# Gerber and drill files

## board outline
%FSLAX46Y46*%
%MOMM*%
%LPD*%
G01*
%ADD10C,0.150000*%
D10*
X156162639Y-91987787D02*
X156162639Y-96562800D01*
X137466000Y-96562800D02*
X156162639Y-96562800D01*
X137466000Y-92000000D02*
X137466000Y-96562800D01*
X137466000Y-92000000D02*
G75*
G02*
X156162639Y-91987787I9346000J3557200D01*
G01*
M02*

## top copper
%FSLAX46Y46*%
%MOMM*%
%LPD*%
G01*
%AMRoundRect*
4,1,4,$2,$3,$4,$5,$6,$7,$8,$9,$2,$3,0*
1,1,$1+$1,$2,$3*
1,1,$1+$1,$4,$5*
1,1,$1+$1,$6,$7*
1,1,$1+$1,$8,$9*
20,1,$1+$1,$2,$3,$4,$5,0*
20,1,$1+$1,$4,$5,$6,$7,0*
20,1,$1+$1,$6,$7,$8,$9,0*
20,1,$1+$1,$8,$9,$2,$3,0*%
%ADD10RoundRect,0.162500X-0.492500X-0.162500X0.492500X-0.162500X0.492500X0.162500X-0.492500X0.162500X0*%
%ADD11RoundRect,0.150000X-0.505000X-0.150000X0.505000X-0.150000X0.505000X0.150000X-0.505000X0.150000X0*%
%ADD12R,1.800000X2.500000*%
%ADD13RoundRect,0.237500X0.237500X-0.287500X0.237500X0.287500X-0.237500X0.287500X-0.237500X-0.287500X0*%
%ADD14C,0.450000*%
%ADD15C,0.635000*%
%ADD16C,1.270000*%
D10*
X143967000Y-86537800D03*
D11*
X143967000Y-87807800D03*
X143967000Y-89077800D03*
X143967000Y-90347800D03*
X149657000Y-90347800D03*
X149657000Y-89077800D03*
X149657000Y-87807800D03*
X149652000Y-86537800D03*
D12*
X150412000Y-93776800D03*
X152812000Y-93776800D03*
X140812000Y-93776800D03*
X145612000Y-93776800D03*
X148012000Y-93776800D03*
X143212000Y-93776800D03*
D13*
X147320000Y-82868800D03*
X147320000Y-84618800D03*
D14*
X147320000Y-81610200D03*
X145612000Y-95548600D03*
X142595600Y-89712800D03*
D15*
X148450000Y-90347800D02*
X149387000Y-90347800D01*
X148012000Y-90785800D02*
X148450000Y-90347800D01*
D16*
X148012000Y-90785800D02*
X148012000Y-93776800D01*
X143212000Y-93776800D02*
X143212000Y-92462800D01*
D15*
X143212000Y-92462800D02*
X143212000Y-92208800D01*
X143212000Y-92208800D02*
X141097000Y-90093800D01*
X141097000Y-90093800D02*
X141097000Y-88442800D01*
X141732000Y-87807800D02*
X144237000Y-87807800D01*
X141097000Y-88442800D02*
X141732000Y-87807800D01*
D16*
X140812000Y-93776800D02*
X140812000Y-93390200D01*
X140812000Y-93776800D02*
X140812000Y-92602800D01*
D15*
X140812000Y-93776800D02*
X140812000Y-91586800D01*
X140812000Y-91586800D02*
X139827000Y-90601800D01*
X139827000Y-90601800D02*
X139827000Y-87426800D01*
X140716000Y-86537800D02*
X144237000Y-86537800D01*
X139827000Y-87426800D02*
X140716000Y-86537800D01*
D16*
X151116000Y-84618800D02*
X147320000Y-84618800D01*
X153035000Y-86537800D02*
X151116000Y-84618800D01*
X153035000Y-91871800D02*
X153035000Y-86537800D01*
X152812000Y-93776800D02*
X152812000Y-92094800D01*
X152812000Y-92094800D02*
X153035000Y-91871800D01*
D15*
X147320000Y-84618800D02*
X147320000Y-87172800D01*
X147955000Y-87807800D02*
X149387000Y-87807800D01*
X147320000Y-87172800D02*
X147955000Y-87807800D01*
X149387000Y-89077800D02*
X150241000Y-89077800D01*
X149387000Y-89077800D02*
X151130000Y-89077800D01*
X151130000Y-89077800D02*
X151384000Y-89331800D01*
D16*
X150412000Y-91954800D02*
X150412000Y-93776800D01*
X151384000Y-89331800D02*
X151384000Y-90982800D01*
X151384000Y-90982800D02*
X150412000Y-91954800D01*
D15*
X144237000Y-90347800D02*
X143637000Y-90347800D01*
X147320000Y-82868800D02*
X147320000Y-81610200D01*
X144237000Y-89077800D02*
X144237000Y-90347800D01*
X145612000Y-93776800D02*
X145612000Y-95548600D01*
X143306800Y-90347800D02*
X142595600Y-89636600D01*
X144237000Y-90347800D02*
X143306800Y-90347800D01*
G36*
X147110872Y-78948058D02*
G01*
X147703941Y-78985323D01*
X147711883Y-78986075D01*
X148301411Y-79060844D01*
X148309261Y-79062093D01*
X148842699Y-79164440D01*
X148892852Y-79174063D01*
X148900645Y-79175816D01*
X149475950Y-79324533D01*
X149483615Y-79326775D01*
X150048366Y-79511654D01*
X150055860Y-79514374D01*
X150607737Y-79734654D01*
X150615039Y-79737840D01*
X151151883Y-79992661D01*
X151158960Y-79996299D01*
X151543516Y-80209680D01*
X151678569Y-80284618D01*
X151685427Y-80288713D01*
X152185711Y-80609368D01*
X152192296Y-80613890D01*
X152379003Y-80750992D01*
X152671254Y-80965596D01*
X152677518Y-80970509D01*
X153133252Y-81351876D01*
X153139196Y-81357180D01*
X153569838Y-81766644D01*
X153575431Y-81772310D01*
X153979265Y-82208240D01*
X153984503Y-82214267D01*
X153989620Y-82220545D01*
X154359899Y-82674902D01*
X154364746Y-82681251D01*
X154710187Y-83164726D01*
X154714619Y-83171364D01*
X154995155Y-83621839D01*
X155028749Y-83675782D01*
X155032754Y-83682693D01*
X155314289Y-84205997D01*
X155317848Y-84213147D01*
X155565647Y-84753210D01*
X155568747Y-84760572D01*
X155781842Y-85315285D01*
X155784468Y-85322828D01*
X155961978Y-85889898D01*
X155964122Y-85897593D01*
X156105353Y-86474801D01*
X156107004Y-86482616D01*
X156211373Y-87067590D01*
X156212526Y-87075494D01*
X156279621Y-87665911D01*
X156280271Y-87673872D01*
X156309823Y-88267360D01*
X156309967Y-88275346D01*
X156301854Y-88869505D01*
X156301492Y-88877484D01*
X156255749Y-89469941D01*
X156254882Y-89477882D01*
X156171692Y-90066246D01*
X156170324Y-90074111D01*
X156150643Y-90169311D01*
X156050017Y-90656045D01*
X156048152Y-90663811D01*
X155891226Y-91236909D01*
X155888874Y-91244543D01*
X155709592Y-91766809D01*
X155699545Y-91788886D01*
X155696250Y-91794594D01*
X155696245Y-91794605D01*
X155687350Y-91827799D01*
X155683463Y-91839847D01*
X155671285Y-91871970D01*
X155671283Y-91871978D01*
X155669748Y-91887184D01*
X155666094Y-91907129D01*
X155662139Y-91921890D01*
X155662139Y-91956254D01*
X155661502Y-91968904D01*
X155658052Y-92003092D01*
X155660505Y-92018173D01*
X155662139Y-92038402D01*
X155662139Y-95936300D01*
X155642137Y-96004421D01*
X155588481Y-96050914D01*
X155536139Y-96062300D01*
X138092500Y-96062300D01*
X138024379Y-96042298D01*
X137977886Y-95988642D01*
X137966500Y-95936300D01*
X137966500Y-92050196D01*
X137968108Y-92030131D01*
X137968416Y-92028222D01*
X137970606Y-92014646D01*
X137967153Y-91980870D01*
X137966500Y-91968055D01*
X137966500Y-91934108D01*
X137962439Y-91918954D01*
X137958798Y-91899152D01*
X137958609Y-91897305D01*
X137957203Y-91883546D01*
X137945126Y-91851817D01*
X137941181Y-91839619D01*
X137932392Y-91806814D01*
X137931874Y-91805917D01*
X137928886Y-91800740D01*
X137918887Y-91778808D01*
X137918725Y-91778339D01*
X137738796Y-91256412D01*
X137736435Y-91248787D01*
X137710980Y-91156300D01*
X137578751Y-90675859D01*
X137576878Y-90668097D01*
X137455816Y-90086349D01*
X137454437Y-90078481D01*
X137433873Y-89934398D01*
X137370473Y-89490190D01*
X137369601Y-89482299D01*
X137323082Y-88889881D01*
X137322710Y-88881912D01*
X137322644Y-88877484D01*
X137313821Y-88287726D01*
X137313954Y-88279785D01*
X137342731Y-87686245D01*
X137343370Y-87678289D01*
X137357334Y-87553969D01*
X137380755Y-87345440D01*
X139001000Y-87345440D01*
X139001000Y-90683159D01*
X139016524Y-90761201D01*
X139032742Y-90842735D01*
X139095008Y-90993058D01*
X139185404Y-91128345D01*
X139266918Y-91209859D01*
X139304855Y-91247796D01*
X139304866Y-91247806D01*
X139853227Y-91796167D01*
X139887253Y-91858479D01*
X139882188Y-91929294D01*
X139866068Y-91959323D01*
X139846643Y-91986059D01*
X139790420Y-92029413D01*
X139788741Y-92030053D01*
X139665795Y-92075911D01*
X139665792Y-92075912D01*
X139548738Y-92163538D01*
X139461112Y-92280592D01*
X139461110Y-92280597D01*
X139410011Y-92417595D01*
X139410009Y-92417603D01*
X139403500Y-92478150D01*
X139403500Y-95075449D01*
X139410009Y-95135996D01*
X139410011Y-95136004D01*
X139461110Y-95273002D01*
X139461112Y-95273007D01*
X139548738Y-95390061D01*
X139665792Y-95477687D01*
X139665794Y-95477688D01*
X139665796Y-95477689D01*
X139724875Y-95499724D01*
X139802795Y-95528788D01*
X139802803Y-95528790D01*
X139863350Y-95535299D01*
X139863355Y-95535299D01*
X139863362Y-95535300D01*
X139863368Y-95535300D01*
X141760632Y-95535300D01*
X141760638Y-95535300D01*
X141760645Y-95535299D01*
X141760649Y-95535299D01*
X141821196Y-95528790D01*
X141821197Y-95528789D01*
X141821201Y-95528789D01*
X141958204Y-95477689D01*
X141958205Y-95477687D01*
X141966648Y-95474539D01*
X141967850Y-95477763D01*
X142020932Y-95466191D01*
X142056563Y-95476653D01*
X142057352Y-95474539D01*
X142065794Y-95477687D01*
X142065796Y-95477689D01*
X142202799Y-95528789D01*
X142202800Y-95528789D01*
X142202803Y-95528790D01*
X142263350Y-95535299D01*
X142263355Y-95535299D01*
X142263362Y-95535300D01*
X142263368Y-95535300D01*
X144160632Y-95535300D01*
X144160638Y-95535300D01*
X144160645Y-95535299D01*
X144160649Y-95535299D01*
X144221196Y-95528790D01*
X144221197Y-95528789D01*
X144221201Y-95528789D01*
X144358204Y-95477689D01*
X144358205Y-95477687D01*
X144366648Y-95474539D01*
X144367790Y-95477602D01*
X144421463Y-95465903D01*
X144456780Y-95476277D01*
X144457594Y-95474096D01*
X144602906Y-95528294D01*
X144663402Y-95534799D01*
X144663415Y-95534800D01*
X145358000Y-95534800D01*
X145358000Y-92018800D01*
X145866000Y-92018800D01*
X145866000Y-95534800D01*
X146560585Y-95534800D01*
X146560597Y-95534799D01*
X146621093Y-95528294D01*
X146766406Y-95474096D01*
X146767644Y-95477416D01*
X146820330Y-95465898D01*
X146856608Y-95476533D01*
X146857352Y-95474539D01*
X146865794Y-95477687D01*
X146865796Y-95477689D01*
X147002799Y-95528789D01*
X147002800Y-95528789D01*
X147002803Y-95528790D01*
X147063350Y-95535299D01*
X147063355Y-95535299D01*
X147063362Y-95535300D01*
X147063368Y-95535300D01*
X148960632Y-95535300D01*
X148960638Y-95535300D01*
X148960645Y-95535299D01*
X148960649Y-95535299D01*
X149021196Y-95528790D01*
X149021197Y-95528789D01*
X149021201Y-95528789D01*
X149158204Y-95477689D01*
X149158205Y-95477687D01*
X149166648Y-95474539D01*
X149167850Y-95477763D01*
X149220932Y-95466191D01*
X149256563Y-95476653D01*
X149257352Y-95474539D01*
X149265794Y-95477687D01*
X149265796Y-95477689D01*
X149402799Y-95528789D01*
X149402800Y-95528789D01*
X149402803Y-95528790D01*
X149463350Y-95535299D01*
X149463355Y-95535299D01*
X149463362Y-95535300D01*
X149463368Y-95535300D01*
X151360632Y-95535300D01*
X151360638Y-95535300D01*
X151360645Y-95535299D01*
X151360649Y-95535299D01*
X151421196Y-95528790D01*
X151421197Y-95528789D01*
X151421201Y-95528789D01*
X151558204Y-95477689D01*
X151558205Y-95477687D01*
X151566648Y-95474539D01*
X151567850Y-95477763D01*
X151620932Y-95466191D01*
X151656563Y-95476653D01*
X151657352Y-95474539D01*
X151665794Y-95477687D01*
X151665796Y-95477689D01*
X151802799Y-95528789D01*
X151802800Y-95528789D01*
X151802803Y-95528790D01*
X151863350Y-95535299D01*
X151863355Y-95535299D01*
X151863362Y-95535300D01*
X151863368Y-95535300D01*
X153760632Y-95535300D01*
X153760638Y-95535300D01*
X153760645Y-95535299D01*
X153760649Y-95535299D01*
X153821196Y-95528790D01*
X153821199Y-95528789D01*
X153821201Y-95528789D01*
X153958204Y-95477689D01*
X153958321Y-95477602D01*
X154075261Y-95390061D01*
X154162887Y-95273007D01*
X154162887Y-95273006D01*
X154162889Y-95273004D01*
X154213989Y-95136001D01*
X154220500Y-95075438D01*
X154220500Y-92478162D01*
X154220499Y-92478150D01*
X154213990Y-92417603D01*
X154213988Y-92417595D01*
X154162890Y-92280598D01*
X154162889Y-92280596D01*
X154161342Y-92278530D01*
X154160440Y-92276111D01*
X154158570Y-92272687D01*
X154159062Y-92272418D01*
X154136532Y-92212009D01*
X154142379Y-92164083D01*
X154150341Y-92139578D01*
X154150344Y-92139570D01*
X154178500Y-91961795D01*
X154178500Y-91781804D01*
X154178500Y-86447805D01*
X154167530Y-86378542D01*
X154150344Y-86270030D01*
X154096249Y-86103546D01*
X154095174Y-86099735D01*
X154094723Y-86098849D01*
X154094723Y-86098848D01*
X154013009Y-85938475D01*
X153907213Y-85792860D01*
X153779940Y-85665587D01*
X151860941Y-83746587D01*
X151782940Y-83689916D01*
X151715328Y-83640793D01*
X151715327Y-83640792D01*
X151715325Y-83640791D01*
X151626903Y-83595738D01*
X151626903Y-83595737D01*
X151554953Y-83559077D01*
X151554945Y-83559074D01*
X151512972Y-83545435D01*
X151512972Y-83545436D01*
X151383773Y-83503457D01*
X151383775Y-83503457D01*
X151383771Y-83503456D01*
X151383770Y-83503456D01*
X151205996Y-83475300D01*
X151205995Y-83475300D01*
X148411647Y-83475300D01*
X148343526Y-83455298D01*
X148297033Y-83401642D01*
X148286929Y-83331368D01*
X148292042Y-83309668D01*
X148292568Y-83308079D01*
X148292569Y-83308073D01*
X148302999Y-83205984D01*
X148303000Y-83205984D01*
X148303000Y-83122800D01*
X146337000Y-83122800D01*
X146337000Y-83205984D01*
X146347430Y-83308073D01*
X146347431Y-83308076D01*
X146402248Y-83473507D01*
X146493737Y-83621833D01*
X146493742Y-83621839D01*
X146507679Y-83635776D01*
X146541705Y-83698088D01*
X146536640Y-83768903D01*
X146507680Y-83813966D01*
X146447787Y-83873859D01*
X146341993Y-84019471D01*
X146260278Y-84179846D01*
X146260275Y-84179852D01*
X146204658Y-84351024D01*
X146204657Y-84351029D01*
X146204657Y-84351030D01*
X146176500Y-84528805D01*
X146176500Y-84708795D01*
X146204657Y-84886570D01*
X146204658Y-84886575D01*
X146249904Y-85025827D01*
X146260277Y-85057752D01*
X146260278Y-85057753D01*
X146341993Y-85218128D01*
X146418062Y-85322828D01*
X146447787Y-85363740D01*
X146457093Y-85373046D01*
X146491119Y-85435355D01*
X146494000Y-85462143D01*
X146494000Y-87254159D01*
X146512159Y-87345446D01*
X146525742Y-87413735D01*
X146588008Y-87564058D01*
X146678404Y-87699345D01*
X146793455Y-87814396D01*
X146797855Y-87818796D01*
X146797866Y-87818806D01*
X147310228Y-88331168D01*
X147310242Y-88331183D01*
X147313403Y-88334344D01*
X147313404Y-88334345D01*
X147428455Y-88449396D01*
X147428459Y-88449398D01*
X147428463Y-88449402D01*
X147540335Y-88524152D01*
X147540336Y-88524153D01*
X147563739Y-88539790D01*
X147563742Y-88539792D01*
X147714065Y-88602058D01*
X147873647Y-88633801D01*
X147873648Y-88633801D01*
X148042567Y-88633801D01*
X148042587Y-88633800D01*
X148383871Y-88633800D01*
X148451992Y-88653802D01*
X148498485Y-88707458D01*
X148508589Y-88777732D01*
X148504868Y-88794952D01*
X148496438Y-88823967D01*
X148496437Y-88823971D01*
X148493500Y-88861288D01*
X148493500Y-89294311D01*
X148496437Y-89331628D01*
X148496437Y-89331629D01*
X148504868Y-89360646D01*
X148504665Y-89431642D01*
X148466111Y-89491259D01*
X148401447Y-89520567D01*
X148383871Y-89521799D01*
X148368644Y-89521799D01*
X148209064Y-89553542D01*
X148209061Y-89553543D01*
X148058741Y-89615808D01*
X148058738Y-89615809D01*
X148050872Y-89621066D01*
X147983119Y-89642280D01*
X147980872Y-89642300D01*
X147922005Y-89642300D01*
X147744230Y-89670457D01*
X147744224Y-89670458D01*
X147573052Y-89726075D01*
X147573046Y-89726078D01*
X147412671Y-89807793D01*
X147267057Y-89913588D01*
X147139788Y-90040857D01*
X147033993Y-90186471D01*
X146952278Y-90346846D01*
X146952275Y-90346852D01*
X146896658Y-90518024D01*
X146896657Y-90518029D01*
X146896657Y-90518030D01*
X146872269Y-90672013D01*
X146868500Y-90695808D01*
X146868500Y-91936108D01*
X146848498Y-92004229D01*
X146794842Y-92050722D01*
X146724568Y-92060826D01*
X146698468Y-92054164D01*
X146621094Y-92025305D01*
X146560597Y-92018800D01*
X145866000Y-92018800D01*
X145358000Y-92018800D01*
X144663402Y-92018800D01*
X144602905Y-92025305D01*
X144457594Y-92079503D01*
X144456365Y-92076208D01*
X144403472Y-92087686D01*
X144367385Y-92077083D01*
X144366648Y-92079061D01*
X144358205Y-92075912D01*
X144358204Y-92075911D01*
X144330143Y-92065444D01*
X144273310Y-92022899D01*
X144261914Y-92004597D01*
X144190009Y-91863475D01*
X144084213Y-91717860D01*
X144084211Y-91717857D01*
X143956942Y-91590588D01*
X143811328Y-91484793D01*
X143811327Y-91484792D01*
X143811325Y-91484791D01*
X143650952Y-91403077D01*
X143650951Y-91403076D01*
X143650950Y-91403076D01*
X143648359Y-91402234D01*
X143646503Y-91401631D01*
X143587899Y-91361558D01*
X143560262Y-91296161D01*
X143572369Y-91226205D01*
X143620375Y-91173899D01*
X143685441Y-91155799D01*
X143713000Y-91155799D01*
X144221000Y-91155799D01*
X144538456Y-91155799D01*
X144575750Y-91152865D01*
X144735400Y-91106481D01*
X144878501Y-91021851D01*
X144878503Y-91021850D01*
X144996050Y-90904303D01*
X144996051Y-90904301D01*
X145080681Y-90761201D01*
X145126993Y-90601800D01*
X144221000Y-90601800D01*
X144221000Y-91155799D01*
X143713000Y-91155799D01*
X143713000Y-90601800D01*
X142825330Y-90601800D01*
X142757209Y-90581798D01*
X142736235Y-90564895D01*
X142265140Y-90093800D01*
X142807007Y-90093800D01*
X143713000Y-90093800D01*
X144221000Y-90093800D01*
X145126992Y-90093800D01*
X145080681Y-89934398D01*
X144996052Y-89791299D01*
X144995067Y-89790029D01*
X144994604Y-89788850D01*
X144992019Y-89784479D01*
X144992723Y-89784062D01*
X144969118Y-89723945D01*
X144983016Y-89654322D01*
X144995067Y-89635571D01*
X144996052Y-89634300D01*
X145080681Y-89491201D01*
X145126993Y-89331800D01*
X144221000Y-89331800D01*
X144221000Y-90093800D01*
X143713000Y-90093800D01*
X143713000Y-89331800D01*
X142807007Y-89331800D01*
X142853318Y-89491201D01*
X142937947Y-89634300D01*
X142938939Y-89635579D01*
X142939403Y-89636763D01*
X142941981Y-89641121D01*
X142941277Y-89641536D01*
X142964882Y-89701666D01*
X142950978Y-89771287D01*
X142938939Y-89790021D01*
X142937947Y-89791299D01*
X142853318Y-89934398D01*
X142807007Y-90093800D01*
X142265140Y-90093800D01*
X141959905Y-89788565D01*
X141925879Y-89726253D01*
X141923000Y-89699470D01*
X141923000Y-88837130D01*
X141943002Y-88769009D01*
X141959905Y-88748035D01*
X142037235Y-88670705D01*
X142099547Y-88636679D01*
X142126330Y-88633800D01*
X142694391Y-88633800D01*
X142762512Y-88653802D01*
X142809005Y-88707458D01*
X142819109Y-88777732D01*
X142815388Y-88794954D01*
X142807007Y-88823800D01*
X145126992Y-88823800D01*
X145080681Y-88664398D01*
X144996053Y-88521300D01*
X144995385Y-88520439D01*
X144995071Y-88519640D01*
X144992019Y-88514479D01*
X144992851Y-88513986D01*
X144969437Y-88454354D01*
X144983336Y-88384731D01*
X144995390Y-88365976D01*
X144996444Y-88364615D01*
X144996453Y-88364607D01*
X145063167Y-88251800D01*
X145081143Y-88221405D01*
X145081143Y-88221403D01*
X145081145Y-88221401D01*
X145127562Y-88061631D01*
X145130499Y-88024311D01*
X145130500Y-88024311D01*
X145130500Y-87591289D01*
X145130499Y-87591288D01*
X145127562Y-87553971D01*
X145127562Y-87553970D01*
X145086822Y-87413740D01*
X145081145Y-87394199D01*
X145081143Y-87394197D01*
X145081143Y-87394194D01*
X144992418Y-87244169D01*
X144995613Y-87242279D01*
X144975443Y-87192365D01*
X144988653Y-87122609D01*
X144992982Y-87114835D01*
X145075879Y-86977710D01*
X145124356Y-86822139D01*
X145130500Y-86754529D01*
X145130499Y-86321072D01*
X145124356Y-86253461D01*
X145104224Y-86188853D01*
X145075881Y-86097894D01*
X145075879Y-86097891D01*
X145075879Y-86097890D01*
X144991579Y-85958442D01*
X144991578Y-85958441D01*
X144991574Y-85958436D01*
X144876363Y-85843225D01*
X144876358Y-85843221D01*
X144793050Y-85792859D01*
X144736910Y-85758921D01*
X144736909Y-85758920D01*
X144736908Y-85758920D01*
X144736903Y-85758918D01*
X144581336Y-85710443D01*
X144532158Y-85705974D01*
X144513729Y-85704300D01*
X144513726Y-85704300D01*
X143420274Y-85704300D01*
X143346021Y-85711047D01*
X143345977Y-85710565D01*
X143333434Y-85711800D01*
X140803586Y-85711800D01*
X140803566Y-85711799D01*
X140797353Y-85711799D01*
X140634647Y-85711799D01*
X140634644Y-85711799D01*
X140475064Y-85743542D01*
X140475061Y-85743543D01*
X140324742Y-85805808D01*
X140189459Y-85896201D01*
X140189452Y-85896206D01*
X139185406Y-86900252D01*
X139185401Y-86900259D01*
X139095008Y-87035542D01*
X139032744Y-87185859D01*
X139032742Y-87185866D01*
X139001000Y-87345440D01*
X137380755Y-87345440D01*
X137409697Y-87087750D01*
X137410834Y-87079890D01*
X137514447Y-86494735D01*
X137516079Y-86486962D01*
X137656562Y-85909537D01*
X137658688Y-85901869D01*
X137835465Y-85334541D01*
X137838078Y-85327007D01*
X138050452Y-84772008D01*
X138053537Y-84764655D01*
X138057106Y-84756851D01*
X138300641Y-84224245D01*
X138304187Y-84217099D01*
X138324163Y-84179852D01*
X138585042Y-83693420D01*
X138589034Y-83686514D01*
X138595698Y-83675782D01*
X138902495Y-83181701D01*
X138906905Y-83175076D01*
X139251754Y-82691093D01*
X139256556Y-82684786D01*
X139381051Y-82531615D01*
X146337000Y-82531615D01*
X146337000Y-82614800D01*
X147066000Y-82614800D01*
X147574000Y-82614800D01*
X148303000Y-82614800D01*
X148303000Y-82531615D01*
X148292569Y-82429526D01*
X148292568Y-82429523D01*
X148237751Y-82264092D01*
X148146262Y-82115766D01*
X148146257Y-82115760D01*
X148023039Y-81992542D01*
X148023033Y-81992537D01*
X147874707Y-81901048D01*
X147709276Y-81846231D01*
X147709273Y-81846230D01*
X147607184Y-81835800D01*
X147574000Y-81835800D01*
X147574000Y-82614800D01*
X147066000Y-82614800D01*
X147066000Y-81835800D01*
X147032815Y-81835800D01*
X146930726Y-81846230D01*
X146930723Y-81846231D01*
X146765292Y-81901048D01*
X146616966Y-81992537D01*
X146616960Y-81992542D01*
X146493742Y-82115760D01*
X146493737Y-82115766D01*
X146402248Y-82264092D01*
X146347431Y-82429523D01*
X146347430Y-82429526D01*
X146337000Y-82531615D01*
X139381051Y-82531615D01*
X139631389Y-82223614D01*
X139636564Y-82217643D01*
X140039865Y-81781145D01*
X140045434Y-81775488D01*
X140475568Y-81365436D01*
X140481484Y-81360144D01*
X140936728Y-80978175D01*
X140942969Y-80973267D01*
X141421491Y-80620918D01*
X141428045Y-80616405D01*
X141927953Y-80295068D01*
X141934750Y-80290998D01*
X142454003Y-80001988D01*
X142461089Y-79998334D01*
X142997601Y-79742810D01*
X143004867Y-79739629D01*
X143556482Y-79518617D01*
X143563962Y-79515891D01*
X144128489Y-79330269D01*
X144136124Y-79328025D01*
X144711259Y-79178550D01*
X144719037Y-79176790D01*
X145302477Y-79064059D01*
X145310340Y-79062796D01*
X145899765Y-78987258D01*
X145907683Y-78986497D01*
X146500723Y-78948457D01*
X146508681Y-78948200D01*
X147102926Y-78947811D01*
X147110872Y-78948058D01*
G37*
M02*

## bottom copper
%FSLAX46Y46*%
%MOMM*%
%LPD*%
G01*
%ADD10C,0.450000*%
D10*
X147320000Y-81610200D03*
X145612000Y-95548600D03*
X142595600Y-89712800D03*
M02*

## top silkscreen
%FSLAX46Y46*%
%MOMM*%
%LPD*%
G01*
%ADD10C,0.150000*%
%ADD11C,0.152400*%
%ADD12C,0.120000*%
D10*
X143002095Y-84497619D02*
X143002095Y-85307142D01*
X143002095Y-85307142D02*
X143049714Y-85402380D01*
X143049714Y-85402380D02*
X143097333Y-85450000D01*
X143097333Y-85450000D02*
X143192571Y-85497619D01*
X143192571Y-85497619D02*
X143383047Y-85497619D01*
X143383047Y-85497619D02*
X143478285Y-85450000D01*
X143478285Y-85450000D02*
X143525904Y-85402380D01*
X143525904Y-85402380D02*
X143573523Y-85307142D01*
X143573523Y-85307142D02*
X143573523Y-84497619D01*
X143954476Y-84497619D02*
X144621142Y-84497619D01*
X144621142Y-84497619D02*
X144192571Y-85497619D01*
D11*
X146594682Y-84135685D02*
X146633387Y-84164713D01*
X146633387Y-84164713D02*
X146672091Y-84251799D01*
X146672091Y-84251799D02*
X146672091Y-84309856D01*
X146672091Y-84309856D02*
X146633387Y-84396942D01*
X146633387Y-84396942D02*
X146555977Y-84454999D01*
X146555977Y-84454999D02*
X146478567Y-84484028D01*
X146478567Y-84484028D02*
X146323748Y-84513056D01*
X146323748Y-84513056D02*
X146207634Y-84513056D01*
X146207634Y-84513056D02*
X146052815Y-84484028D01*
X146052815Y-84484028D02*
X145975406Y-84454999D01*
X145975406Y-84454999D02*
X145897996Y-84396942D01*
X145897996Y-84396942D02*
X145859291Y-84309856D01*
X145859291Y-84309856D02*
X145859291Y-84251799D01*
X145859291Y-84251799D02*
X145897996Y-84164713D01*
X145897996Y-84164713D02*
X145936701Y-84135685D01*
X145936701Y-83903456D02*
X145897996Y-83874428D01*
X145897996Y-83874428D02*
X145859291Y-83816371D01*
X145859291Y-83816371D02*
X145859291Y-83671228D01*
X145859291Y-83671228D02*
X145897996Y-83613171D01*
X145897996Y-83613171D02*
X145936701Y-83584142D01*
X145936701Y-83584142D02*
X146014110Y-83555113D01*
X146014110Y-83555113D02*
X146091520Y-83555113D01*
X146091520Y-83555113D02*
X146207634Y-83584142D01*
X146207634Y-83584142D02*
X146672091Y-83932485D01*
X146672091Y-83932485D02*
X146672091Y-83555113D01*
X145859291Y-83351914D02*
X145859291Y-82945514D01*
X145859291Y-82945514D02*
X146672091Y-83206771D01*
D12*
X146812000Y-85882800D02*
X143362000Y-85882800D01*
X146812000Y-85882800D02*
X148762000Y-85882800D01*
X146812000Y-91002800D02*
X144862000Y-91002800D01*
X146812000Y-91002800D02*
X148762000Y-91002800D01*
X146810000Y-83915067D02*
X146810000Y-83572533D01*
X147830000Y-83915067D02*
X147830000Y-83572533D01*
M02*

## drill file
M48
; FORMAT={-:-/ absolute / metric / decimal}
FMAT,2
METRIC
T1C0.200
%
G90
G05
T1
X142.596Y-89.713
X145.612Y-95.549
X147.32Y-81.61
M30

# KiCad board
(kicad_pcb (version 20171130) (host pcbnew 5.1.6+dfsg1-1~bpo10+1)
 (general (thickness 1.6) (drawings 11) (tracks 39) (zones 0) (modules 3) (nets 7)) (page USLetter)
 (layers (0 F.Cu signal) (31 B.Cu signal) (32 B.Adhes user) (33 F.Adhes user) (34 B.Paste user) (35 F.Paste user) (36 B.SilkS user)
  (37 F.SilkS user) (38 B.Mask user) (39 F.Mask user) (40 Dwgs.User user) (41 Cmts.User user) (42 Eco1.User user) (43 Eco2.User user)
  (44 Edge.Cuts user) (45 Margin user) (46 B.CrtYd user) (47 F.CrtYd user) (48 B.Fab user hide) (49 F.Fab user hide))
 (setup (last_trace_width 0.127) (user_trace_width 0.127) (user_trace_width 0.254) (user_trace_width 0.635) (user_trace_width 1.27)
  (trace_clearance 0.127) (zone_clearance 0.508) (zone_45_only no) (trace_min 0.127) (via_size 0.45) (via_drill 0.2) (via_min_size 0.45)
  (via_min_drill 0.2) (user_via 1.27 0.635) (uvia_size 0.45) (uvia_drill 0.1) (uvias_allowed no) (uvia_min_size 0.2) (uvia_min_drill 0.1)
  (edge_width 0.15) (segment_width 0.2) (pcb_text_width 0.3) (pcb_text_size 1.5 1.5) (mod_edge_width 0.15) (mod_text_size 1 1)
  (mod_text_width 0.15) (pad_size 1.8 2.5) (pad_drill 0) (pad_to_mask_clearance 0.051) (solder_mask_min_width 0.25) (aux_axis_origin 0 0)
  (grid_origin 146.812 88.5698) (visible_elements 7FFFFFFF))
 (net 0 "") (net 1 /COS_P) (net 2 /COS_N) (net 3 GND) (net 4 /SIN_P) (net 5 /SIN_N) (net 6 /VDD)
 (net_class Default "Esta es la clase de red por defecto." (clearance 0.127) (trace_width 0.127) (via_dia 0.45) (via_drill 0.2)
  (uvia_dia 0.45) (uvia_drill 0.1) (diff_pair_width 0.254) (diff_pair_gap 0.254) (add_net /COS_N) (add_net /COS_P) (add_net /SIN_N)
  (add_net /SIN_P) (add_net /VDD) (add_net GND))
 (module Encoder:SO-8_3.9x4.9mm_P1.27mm (layer F.Cu) (at 146.812 88.4428)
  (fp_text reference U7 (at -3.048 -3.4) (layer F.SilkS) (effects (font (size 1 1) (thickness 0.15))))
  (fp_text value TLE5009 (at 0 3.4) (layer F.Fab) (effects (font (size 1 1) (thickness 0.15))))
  (fp_line (start 0 -2.56) (end -3.45 -2.56) (layer F.SilkS) (width 0.12))
  (fp_line (start 0 -2.56) (end 1.95 -2.56) (layer F.SilkS) (width 0.12))
  (fp_line (start 0 2.56) (end -1.95 2.56) (layer F.SilkS) (width 0.12))
  (fp_line (start 0 2.56) (end 1.95 2.56) (layer F.SilkS) (width 0.12))
  (pad 1 smd roundrect (at -2.845 -1.905) (size 1.31 0.65) (layers F.Cu F.Paste F.Mask) (roundrect_rratio 0.25) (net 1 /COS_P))
  (pad 2 smd roundrect (at -2.845 -0.635) (size 1.31 0.6) (layers F.Cu F.Paste F.Mask) (roundrect_rratio 0.25) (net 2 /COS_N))
  (pad 3 smd roundrect (at -2.845 0.635) (size 1.31 0.6) (layers F.Cu F.Paste F.Mask) (roundrect_rratio 0.25) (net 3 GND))
  (pad 4 smd roundrect (at -2.845 1.905) (size 1.31 0.6) (layers F.Cu F.Paste F.Mask) (roundrect_rratio 0.25) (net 3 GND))
  (pad 5 smd roundrect (at 2.845 1.905) (size 1.31 0.6) (layers F.Cu F.Paste F.Mask) (roundrect_rratio 0.25) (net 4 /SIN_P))
  (pad 6 smd roundrect (at 2.845 0.635) (size 1.31 0.6) (layers F.Cu F.Paste F.Mask) (roundrect_rratio 0.25) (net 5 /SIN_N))
  (pad 7 smd roundrect (at 2.845 -0.635) (size 1.31 0.6) (layers F.Cu F.Paste F.Mask) (roundrect_rratio 0.25) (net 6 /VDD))
  (pad 8 smd roundrect (at 2.84 -1.905) (size 1.31 0.6) (layers F.Cu F.Paste F.Mask) (roundrect_rratio 0.25)))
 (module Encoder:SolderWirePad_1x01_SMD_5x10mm (layer F.Cu) (at 146.812 93.7768)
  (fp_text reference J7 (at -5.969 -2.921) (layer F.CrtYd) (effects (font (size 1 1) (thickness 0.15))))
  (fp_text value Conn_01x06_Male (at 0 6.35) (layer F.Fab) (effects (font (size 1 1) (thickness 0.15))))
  (pad 5 smd rect (at 3.6 0) (size 1.8 2.5) (layers F.Cu F.Paste F.Mask) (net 5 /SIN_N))
  (pad 6 smd rect (at 6 0) (size 1.8 2.5) (layers F.Cu F.Paste F.Mask) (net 6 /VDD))
  (pad 1 smd rect (at -6 0) (size 1.8 2.5) (layers F.Cu F.Paste F.Mask) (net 1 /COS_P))
  (pad 3 smd rect (at -1.2 0) (size 1.8 2.5) (layers F.Cu F.Paste F.Mask) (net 3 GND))
  (pad 4 smd rect (at 1.2 0) (size 1.8 2.5) (layers F.Cu F.Paste F.Mask) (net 4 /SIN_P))
  (pad 2 smd rect (at -3.6 0) (size 1.8 2.5) (layers F.Cu F.Paste F.Mask) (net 2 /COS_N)))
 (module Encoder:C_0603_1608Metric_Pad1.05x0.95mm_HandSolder (layer F.Cu) (at 147.32 83.7438 90)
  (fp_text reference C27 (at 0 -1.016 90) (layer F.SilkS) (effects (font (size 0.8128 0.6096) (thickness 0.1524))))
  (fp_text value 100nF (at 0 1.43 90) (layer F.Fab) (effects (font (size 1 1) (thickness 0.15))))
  (fp_line (start -0.171267 -0.51) (end 0.171267 -0.51) (layer F.SilkS) (width 0.12))
  (fp_line (start -0.171267 0.51) (end 0.171267 0.51) (layer F.SilkS) (width 0.12))
  (pad 2 smd roundrect (at 0.875 0 90) (size 1.05 0.95) (layers F.Cu F.Paste F.Mask) (roundrect_rratio 0.25) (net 3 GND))
  (pad 1 smd roundrect (at -0.875 0 90) (size 1.05 0.95) (layers F.Cu F.Paste F.Mask) (roundrect_rratio 0.25) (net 6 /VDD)))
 (gr_line (start 156.162639 91.987787) (end 156.162639 96.5628) (layer Edge.Cuts) (width 0.15))
 (gr_line (start 137.466 96.5628) (end 156.162639 96.5628) (layer Edge.Cuts) (width 0.15))
 (gr_line (start 137.466 92) (end 137.466 96.5628) (layer Edge.Cuts) (width 0.15))
 (gr_arc (start 146.812 88.4428) (end 137.466 92) (angle 221.6) (layer Edge.Cuts) (width 0.15))
 (segment (start 148.45 90.3478) (end 149.387 90.3478) (width 0.635) (layer F.Cu) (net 4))
 (segment (start 148.012 90.7858) (end 148.45 90.3478) (width 0.635) (layer F.Cu) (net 4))
 (segment (start 148.012 90.7858) (end 148.012 93.7768) (width 1.27) (layer F.Cu) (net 4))
 (segment (start 143.212 93.7768) (end 143.212 92.4628) (width 1.27) (layer F.Cu) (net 2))
 (segment (start 143.212 92.4628) (end 143.212 92.2088) (width 0.635) (layer F.Cu) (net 2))
 (segment (start 143.212 92.2088) (end 141.097 90.0938) (width 0.635) (layer F.Cu) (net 2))
 (segment (start 141.097 90.0938) (end 141.097 88.4428) (width 0.635) (layer F.Cu) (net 2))
 (segment (start 141.732 87.8078) (end 144.237 87.8078) (width 0.635) (layer F.Cu) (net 2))
 (segment (start 141.097 88.4428) (end 141.732 87.8078) (width 0.635) (layer F.Cu) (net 2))
 (segment (start 140.812 93.7768) (end 140.812 93.3902) (width 1.27) (layer F.Cu) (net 1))
 (segment (start 140.812 93.7768) (end 140.812 92.6028) (width 1.27) (layer F.Cu) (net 1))
 (segment (start 140.812 93.7768) (end 140.812 91.5868) (width 0.635) (layer F.Cu) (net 1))
 (segment (start 140.812 91.5868) (end 139.827 90.6018) (width 0.635) (layer F.Cu) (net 1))
 (segment (start 139.827 90.6018) (end 139.827 87.4268) (width 0.635) (layer F.Cu) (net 1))
 (segment (start 140.716 86.5378) (end 144.237 86.5378) (width 0.635) (layer F.Cu) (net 1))
 (segment (start 139.827 87.4268) (end 140.716 86.5378) (width 0.635) (layer F.Cu) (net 1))
 (segment (start 151.116 84.6188) (end 147.32 84.6188) (width 1.27) (layer F.Cu) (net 6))
 (segment (start 153.035 86.5378) (end 151.116 84.6188) (width 1.27) (layer F.Cu) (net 6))
 (segment (start 153.035 91.8718) (end 153.035 86.5378) (width 1.27) (layer F.Cu) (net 6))
 (segment (start 152.812 93.7768) (end 152.812 92.0948) (width 1.27) (layer F.Cu) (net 6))
 (segment (start 152.812 92.0948) (end 153.035 91.8718) (width 1.27) (layer F.Cu) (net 6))
 (segment (start 147.32 84.6188) (end 147.32 87.1728) (width 0.635) (layer F.Cu) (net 6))
 (segment (start 147.955 87.8078) (end 149.387 87.8078) (width 0.635) (layer F.Cu) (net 6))
 (segment (start 147.32 87.1728) (end 147.955 87.8078) (width 0.635) (layer F.Cu) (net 6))
 (segment (start 149.387 89.0778) (end 150.241 89.0778) (width 0.635) (layer F.Cu) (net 5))
 (segment (start 149.387 89.0778) (end 151.13 89.0778) (width 0.635) (layer F.Cu) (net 5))
 (segment (start 151.13 89.0778) (end 151.384 89.3318) (width 0.635) (layer F.Cu) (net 5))
 (segment (start 150.412 91.9548) (end 150.412 93.7768) (width 1.27) (layer F.Cu) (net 5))
 (segment (start 151.384 89.3318) (end 151.384 90.9828) (width 1.27) (layer F.Cu) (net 5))
 (segment (start 151.384 90.9828) (end 150.412 91.9548) (width 1.27) (layer F.Cu) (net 5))
 (segment (start 144.237 90.3478) (end 143.637 90.3478) (width 0.635) (layer F.Cu) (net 3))
 (segment (start 147.32 82.8688) (end 147.32 81.6102) (width 0.635) (layer F.Cu) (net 3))
 (via (at 147.32 81.6102) (size 0.45) (drill 0.2) (layers F.Cu B.Cu) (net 3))
 (segment (start 144.237 89.0778) (end 144.237 90.3478) (width 0.635) (layer F.Cu) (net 3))
 (segment (start 145.612 93.7768) (end 145.612 95.5486) (width 0.635) (layer F.Cu) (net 3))
 (via (at 145.612 95.5486) (size 0.45) (drill 0.2) (layers F.Cu B.Cu) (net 3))
 (via (at 142.5956 89.7128) (size 0.45) (drill 0.2) (layers F.Cu B.Cu) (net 3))
 (segment (start 143.3068 90.3478) (end 142.5956 89.6366) (width 0.635) (layer F.Cu) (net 3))
 (segment (start 144.237 90.3478) (end 143.3068 90.3478) (width 0.635) (layer F.Cu) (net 3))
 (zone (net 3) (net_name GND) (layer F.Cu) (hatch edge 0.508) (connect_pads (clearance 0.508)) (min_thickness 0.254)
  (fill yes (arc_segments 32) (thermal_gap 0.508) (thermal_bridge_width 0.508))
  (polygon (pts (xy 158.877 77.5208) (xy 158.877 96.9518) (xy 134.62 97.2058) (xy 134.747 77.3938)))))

